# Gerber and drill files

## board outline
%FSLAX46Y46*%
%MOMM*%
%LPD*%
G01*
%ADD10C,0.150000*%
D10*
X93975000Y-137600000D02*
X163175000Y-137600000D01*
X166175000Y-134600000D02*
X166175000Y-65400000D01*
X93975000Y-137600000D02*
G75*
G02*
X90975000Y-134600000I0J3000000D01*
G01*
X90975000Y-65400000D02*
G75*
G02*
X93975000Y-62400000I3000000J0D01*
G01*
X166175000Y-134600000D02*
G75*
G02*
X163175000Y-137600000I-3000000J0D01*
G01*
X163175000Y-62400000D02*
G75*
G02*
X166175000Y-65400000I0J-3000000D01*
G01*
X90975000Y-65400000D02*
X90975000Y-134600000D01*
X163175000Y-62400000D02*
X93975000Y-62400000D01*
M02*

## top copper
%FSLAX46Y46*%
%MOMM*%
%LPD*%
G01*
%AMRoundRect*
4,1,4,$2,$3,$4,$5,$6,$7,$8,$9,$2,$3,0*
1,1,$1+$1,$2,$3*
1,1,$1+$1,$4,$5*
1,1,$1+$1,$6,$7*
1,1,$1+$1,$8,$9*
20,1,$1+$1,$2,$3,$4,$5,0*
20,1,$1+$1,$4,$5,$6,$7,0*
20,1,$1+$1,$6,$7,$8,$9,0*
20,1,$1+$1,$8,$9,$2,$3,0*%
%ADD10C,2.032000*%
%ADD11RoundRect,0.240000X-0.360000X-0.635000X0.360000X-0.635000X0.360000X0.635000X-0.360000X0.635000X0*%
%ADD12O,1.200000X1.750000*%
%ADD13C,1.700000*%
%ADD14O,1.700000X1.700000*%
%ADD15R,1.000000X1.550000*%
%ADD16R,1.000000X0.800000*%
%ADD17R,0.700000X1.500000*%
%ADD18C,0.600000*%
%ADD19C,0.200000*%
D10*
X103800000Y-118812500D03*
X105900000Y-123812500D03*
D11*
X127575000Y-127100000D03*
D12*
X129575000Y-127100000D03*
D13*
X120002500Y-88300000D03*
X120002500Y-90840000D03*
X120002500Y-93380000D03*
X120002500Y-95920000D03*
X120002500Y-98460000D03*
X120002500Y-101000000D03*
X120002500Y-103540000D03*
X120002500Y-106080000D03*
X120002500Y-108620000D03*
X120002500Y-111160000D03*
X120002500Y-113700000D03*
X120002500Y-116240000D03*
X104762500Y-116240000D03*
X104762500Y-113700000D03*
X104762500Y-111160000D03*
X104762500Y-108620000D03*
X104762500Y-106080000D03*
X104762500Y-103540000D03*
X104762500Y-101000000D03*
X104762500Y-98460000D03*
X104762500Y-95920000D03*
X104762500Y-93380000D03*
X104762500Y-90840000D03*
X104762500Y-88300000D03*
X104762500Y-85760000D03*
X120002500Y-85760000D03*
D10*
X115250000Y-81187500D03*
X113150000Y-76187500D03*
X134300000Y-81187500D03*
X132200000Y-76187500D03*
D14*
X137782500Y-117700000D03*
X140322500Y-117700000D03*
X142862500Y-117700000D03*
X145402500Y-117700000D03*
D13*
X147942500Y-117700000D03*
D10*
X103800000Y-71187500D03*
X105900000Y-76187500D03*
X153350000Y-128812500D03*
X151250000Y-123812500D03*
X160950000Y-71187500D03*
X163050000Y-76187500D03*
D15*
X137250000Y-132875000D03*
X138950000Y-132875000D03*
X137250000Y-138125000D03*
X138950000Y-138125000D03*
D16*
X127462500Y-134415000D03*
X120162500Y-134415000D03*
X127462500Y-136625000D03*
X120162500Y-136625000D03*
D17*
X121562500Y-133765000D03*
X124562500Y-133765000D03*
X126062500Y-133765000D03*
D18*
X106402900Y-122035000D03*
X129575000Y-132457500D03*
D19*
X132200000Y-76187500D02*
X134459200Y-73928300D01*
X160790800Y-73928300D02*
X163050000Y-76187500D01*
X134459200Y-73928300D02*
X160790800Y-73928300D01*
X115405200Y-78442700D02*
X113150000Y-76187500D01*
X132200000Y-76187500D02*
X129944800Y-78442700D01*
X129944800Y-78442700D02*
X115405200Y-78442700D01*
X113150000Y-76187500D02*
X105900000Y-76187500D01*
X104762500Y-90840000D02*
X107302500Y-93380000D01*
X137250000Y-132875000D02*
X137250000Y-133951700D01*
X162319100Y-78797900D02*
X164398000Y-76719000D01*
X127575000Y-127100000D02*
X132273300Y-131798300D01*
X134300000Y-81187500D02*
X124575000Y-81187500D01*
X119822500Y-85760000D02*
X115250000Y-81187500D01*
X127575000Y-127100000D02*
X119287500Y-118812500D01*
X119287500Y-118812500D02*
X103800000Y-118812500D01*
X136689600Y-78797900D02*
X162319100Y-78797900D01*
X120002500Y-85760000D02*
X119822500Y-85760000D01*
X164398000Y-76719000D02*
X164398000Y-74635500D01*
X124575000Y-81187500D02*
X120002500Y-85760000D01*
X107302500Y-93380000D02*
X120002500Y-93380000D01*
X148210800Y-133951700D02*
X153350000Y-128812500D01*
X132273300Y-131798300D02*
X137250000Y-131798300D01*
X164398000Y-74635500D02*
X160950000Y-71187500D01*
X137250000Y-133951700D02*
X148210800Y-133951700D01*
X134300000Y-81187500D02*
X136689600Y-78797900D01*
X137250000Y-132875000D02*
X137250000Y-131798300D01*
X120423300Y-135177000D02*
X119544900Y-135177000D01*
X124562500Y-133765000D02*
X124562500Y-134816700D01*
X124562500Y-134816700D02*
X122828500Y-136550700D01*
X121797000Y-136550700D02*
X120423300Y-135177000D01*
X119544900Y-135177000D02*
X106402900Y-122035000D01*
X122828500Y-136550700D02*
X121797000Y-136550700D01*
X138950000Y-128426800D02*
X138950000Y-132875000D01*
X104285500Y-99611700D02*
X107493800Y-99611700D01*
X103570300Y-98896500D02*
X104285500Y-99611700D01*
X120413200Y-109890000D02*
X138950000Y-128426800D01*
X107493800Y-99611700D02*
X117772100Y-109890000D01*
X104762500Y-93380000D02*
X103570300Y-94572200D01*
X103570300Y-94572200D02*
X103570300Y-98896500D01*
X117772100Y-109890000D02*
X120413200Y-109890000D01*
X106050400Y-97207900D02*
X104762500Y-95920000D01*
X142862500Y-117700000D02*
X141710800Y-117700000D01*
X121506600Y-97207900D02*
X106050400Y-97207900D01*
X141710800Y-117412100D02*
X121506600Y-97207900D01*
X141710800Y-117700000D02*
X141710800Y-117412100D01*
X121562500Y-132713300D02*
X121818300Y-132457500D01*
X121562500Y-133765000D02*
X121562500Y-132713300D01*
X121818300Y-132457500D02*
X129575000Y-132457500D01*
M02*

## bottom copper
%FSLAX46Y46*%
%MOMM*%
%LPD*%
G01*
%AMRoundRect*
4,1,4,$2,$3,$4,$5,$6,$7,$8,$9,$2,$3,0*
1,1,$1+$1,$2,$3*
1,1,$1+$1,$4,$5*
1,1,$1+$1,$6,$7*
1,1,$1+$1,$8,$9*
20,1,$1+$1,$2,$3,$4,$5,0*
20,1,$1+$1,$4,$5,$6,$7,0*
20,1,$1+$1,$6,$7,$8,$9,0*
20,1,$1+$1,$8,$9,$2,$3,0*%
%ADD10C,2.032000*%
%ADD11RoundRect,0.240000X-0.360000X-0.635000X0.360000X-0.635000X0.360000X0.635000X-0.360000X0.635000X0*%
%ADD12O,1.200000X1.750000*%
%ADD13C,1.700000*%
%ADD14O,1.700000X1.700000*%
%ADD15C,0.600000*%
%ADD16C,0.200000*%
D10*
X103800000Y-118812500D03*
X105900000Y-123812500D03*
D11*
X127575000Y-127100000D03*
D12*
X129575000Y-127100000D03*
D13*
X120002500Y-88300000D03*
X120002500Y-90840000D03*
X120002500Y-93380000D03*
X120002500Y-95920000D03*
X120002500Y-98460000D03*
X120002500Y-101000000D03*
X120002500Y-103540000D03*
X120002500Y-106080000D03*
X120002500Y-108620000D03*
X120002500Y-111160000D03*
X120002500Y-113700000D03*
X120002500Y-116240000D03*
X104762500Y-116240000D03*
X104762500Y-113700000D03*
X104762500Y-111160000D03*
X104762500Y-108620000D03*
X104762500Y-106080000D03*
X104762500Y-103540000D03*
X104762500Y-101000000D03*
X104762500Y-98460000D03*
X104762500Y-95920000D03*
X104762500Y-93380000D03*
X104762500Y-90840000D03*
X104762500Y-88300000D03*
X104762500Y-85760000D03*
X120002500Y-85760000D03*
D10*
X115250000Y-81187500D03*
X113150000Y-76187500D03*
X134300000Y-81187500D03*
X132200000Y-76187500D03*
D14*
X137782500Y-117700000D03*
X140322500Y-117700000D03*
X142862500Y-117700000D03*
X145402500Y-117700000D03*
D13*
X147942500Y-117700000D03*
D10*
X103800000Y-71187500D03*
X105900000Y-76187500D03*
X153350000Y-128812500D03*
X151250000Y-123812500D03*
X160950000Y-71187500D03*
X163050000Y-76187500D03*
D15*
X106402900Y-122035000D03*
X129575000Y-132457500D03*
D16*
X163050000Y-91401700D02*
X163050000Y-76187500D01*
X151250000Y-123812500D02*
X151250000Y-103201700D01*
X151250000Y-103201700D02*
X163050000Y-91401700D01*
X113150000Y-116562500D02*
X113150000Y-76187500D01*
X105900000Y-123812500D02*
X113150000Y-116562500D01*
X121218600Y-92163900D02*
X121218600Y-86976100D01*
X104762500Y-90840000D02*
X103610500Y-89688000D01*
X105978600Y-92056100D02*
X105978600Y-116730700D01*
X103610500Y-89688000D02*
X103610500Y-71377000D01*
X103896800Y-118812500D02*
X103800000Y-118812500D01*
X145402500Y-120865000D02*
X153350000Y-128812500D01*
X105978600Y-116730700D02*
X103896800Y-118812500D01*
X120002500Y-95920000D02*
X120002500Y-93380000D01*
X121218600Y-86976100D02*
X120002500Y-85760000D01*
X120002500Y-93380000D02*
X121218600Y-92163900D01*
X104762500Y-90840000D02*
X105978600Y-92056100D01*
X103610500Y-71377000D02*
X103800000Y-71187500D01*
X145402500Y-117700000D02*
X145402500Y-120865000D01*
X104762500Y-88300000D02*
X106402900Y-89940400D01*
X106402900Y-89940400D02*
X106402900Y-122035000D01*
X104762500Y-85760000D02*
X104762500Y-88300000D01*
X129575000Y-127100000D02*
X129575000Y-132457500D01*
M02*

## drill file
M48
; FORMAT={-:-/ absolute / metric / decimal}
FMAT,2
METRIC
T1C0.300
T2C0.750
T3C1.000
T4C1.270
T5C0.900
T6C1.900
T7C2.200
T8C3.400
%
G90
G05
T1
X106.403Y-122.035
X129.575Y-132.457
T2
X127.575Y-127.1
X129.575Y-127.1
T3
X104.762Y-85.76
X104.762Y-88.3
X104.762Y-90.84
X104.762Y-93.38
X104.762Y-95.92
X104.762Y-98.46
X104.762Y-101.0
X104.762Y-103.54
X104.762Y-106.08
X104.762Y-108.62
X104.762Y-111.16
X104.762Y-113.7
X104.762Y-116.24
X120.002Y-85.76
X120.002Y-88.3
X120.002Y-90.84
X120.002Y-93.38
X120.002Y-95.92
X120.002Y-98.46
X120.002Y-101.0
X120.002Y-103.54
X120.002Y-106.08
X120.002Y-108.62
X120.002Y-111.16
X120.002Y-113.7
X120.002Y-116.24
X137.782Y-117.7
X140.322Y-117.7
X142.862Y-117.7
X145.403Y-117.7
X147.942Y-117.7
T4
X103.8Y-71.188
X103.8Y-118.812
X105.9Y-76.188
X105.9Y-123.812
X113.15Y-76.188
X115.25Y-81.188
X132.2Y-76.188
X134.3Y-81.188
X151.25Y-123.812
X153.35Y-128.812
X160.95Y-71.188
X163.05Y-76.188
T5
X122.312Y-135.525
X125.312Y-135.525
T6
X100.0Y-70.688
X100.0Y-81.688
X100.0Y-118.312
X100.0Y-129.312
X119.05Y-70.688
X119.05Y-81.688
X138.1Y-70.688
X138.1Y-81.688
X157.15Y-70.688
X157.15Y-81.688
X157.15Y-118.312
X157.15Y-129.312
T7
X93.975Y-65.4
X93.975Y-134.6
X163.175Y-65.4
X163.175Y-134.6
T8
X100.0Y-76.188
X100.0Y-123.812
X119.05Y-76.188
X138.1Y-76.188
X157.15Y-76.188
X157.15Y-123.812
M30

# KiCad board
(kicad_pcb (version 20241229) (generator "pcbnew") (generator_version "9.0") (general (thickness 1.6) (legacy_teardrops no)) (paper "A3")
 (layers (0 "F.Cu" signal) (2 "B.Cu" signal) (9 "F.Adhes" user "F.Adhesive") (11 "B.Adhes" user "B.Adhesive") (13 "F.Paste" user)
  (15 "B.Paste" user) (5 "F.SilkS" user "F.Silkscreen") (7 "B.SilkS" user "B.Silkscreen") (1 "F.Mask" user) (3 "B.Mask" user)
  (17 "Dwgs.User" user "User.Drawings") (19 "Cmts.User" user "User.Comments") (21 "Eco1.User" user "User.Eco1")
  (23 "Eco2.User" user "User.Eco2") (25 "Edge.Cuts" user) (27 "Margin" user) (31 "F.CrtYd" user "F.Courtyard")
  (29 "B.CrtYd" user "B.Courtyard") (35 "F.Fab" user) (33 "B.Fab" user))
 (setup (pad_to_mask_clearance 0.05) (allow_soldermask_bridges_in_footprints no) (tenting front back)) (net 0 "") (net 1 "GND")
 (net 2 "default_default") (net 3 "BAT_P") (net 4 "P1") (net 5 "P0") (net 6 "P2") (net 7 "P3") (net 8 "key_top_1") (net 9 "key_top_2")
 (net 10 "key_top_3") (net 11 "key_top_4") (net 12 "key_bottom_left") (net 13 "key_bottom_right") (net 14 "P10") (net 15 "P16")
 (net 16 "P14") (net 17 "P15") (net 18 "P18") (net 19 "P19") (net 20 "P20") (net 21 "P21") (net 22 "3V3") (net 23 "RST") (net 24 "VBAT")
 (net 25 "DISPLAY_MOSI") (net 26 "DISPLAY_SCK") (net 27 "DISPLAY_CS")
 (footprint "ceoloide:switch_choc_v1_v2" (layer "F.Cu") (at 100 123.8125 -90)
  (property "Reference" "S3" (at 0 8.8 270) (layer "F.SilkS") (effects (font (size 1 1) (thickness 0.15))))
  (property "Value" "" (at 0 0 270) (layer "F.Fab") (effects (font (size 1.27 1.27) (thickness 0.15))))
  (pad "" np_thru_hole circle (at -5.5 0 270) (size 1.9 1.9) (drill 1.9) (layers "*.Cu" "*.Mask"))
  (pad "" np_thru_hole circle (at 0 0 270) (size 3.4 3.4) (drill 3.4) (layers "*.Cu" "*.Mask"))
  (pad "" np_thru_hole circle (at 5.5 0 270) (size 1.9 1.9) (drill 1.9) (layers "*.Cu" "*.Mask"))
  (pad "1" thru_hole circle (at -5 -3.8 105) (size 2.032 2.032) (drill 1.27) (layers "*.Cu" "*.Mask") (remove_unused_layers no)
   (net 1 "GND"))
  (pad "2" thru_hole circle (at 0 -5.9 105) (size 2.032 2.032) (drill 1.27) (layers "*.Cu" "*.Mask") (remove_unused_layers no)
   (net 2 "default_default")))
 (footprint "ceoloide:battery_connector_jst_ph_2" (layer "F.Cu") (at 128.575 127.1)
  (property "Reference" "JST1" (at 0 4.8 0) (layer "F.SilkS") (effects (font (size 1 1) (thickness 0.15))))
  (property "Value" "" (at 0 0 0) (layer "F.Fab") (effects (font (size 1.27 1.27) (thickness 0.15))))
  (pad "1" thru_hole roundrect (at -1 0) (size 1.2 1.75) (drill 0.75) (layers "*.Cu" "*.Mask") (remove_unused_layers no)
   (roundrect_rratio 0.2) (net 1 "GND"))
  (pad "2" thru_hole oval (at 1 0) (size 1.2 1.75) (drill 0.75) (layers "*.Cu" "*.Mask") (remove_unused_layers no) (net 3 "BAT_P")))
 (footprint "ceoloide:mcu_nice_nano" (layer "F.Cu") (at 112.3825 101)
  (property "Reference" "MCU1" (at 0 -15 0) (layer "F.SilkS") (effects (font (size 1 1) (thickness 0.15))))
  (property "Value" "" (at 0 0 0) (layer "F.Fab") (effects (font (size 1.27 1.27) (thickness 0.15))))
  (pad "1" thru_hole circle (at 7.62 -12.7) (size 1.7 1.7) (drill 1) (layers "*.Cu" "*.Mask") (remove_unused_layers no) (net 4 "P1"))
  (pad "2" thru_hole circle (at 7.62 -10.16) (size 1.7 1.7) (drill 1) (layers "*.Cu" "*.Mask") (remove_unused_layers no) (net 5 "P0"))
  (pad "3" thru_hole circle (at 7.62 -7.62) (size 1.7 1.7) (drill 1) (layers "*.Cu" "*.Mask") (remove_unused_layers no) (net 1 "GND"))
  (pad "4" thru_hole circle (at 7.62 -5.08) (size 1.7 1.7) (drill 1) (layers "*.Cu" "*.Mask") (remove_unused_layers no) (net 1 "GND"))
  (pad "5" thru_hole circle (at 7.62 -2.54) (size 1.7 1.7) (drill 1) (layers "*.Cu" "*.Mask") (remove_unused_layers no) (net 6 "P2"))
  (pad "6" thru_hole circle (at 7.62 0) (size 1.7 1.7) (drill 1) (layers "*.Cu" "*.Mask") (remove_unused_layers no) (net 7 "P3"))
  (pad "7" thru_hole circle (at 7.62 2.54) (size 1.7 1.7) (drill 1) (layers "*.Cu" "*.Mask") (remove_unused_layers no) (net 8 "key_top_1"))
  (pad "8" thru_hole circle (at 7.62 5.08) (size 1.7 1.7) (drill 1) (layers "*.Cu" "*.Mask") (remove_unused_layers no) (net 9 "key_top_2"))
  (pad "9" thru_hole circle (at 7.62 7.62) (size 1.7 1.7) (drill 1) (layers "*.Cu" "*.Mask") (remove_unused_layers no) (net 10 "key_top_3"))
  (pad "10" thru_hole circle (at 7.62 10.16) (size 1.7 1.7) (drill 1) (layers "*.Cu" "*.Mask") (remove_unused_layers no)
   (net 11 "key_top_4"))
  (pad "11" thru_hole circle (at 7.62 12.7) (size 1.7 1.7) (drill 1) (layers "*.Cu" "*.Mask") (remove_unused_layers no)
   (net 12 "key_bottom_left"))
  (pad "12" thru_hole circle (at 7.62 15.24) (size 1.7 1.7) (drill 1) (layers "*.Cu" "*.Mask") (remove_unused_layers no)
   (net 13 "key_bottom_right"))
  (pad "13" thru_hole circle (at -7.62 15.24) (size 1.7 1.7) (drill 1) (layers "*.Cu" "*.Mask") (remove_unused_layers no) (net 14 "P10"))
  (pad "14" thru_hole circle (at -7.62 12.7) (size 1.7 1.7) (drill 1) (layers "*.Cu" "*.Mask") (remove_unused_layers no) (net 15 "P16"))
  (pad "15" thru_hole circle (at -7.62 10.16) (size 1.7 1.7) (drill 1) (layers "*.Cu" "*.Mask") (remove_unused_layers no) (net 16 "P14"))
  (pad "16" thru_hole circle (at -7.62 7.62) (size 1.7 1.7) (drill 1) (layers "*.Cu" "*.Mask") (remove_unused_layers no) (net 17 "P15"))
  (pad "17" thru_hole circle (at -7.62 5.08) (size 1.7 1.7) (drill 1) (layers "*.Cu" "*.Mask") (remove_unused_layers no) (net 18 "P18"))
  (pad "18" thru_hole circle (at -7.62 2.54) (size 1.7 1.7) (drill 1) (layers "*.Cu" "*.Mask") (remove_unused_layers no) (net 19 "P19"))
  (pad "19" thru_hole circle (at -7.62 0) (size 1.7 1.7) (drill 1) (layers "*.Cu" "*.Mask") (remove_unused_layers no) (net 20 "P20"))
  (pad "20" thru_hole circle (at -7.62 -2.54) (size 1.7 1.7) (drill 1) (layers "*.Cu" "*.Mask") (remove_unused_layers no) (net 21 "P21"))
  (pad "21" thru_hole circle (at -7.62 -5.08) (size 1.7 1.7) (drill 1) (layers "*.Cu" "*.Mask") (remove_unused_layers no) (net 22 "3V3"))
  (pad "22" thru_hole circle (at -7.62 -7.62) (size 1.7 1.7) (drill 1) (layers "*.Cu" "*.Mask") (remove_unused_layers no) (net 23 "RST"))
  (pad "23" thru_hole circle (at -7.62 -10.16) (size 1.7 1.7) (drill 1) (layers "*.Cu" "*.Mask") (remove_unused_layers no) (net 1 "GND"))
  (pad "24" thru_hole circle (at -7.62 -12.7) (size 1.7 1.7) (drill 1) (layers "*.Cu" "*.Mask") (remove_unused_layers no) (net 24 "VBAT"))
  (pad "25" thru_hole circle (at -7.62 -15.24) (size 1.7 1.7) (drill 1) (layers "*.Cu" "*.Mask") (remove_unused_layers no) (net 24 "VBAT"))
  (pad "26" thru_hole circle (at 7.62 -15.24) (size 1.7 1.7) (drill 1) (layers "*.Cu" "*.Mask") (remove_unused_layers no) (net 1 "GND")))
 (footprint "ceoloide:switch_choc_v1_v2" (layer "F.Cu") (at 119.05 76.1875 90)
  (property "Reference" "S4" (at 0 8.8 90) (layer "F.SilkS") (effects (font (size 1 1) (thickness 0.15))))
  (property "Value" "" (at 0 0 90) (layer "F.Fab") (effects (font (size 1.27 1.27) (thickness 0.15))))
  (pad "" np_thru_hole circle (at -5.5 0 90) (size 1.9 1.9) (drill 1.9) (layers "*.Cu" "*.Mask"))
  (pad "" np_thru_hole circle (at 0 0 90) (size 3.4 3.4) (drill 3.4) (layers "*.Cu" "*.Mask"))
  (pad "" np_thru_hole circle (at 5.5 0 90) (size 1.9 1.9) (drill 1.9) (layers "*.Cu" "*.Mask"))
  (pad "1" thru_hole circle (at -5 -3.8 285) (size 2.032 2.032) (drill 1.27) (layers "*.Cu" "*.Mask") (remove_unused_layers no)
   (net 1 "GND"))
  (pad "2" thru_hole circle (at 0 -5.9 285) (size 2.032 2.032) (drill 1.27) (layers "*.Cu" "*.Mask") (remove_unused_layers no)
   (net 2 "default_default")))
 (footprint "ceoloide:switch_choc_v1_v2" (layer "F.Cu") (at 138.1 76.1875 90)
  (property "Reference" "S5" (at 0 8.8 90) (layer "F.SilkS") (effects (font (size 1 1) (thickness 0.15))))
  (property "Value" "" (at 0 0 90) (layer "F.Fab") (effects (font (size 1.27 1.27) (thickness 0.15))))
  (pad "" np_thru_hole circle (at -5.5 0 90) (size 1.9 1.9) (drill 1.9) (layers "*.Cu" "*.Mask"))
  (pad "" np_thru_hole circle (at 0 0 90) (size 3.4 3.4) (drill 3.4) (layers "*.Cu" "*.Mask"))
  (pad "" np_thru_hole circle (at 5.5 0 90) (size 1.9 1.9) (drill 1.9) (layers "*.Cu" "*.Mask"))
  (pad "1" thru_hole circle (at -5 -3.8 285) (size 2.032 2.032) (drill 1.27) (layers "*.Cu" "*.Mask") (remove_unused_layers no)
   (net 1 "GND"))
  (pad "2" thru_hole circle (at 0 -5.9 285) (size 2.032 2.032) (drill 1.27) (layers "*.Cu" "*.Mask") (remove_unused_layers no)
   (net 2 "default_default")))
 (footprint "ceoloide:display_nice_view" (layer "F.Cu") (at 142.8625 101)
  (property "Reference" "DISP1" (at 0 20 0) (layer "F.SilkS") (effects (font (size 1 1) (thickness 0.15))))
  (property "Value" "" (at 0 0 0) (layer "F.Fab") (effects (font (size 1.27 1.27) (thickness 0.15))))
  (pad "1" thru_hole oval (at -5.08 16.7 270) (size 1.7 1.7) (drill 1) (layers "*.Cu" "*.Mask") (remove_unused_layers no)
   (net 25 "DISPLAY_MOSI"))
  (pad "2" thru_hole oval (at -2.54 16.7 270) (size 1.7 1.7) (drill 1) (layers "*.Cu" "*.Mask") (remove_unused_layers no)
   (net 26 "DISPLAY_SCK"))
  (pad "3" thru_hole oval (at 0 16.7 270) (size 1.7 1.7) (drill 1) (layers "*.Cu" "*.Mask") (remove_unused_layers no) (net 22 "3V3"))
  (pad "4" thru_hole oval (at 2.54 16.7 270) (size 1.7 1.7) (drill 1) (layers "*.Cu" "*.Mask") (remove_unused_layers no) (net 1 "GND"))
  (pad "5" thru_hole circle (at 5.08 16.7 270) (size 1.7 1.7) (drill 1) (layers "*.Cu" "*.Mask") (remove_unused_layers no)
   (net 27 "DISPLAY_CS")))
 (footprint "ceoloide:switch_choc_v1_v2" (layer "F.Cu") (at 100 76.1875 -90)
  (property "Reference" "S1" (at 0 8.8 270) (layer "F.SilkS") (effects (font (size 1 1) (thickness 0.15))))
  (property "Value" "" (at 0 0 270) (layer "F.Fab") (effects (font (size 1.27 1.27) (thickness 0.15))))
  (pad "" np_thru_hole circle (at -5.5 0 270) (size 1.9 1.9) (drill 1.9) (layers "*.Cu" "*.Mask"))
  (pad "" np_thru_hole circle (at 0 0 270) (size 3.4 3.4) (drill 3.4) (layers "*.Cu" "*.Mask"))
  (pad "" np_thru_hole circle (at 5.5 0 270) (size 1.9 1.9) (drill 1.9) (layers "*.Cu" "*.Mask"))
  (pad "1" thru_hole circle (at -5 -3.8 105) (size 2.032 2.032) (drill 1.27) (layers "*.Cu" "*.Mask") (remove_unused_layers no)
   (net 1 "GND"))
  (pad "2" thru_hole circle (at 0 -5.9 105) (size 2.032 2.032) (drill 1.27) (layers "*.Cu" "*.Mask") (remove_unused_layers no)
   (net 2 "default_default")))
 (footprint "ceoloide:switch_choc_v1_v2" (layer "F.Cu") (at 157.15 123.8125 90)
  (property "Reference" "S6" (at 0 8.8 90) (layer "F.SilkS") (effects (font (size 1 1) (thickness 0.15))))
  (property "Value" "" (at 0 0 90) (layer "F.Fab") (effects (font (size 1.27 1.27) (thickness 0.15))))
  (pad "" np_thru_hole circle (at -5.5 0 90) (size 1.9 1.9) (drill 1.9) (layers "*.Cu" "*.Mask"))
  (pad "" np_thru_hole circle (at 0 0 90) (size 3.4 3.4) (drill 3.4) (layers "*.Cu" "*.Mask"))
  (pad "" np_thru_hole circle (at 5.5 0 90) (size 1.9 1.9) (drill 1.9) (layers "*.Cu" "*.Mask"))
  (pad "1" thru_hole circle (at -5 -3.8 285) (size 2.032 2.032) (drill 1.27) (layers "*.Cu" "*.Mask") (remove_unused_layers no)
   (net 1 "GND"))
  (pad "2" thru_hole circle (at 0 -5.9 285) (size 2.032 2.032) (drill 1.27) (layers "*.Cu" "*.Mask") (remove_unused_layers no)
   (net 2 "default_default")))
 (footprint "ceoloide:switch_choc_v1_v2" (layer "F.Cu") (at 157.15 76.1875 -90)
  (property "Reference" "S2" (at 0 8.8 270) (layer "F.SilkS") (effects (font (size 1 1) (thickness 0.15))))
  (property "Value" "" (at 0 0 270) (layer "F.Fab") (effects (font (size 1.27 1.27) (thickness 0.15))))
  (pad "" np_thru_hole circle (at -5.5 0 270) (size 1.9 1.9) (drill 1.9) (layers "*.Cu" "*.Mask"))
  (pad "" np_thru_hole circle (at 0 0 270) (size 3.4 3.4) (drill 3.4) (layers "*.Cu" "*.Mask"))
  (pad "" np_thru_hole circle (at 5.5 0 270) (size 1.9 1.9) (drill 1.9) (layers "*.Cu" "*.Mask"))
  (pad "1" thru_hole circle (at -5 -3.8 105) (size 2.032 2.032) (drill 1.27) (layers "*.Cu" "*.Mask") (remove_unused_layers no)
   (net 1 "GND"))
  (pad "2" thru_hole circle (at 0 -5.9 105) (size 2.032 2.032) (drill 1.27) (layers "*.Cu" "*.Mask") (remove_unused_layers no)
   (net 2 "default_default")))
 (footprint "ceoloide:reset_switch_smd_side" (layer "F.Cu") (at 138.1 135.5 90)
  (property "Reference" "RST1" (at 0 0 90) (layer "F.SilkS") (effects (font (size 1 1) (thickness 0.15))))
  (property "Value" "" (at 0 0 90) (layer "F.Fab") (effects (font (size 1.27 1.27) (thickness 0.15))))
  (pad "1" smd rect (at 2.625 -0.85 270) (size 1.55 1) (layers "F.Cu" "F.Mask" "F.Paste") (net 1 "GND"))
  (pad "2" smd rect (at 2.625 0.85 270) (size 1.55 1) (layers "F.Cu" "F.Mask" "F.Paste") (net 23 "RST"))
  (pad "3" smd rect (at -2.625 -0.85 270) (size 1.55 1) (layers "F.Cu" "F.Mask" "F.Paste") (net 1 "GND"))
  (pad "4" smd rect (at -2.625 0.85 270) (size 1.55 1) (layers "F.Cu" "F.Mask" "F.Paste") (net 23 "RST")))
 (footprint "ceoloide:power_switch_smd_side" (layer "F.Cu") (at 123.8125 135.5 -90)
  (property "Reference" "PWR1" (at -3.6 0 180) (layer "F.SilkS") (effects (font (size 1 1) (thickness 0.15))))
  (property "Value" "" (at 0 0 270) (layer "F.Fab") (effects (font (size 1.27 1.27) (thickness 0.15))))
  (pad "" smd rect (at -1.085 -3.65) (size 1 0.8) (layers "F.Cu" "F.Mask" "F.Paste"))
  (pad "" smd rect (at -1.085 3.65) (size 1 0.8) (layers "F.Cu" "F.Mask" "F.Paste"))
  (pad "" np_thru_hole circle (at 0.025 -1.5) (size 0.9 0.9) (drill 0.9) (layers "*.Cu" "*.Mask"))
  (pad "" np_thru_hole circle (at 0.025 1.5) (size 0.9 0.9) (drill 0.9) (layers "*.Cu" "*.Mask"))
  (pad "" smd rect (at 1.125 -3.65) (size 1 0.8) (layers "F.Cu" "F.Mask" "F.Paste"))
  (pad "" smd rect (at 1.125 3.65) (size 1 0.8) (layers "F.Cu" "F.Mask" "F.Paste"))
  (pad "1" smd rect (at -1.735 2.25) (size 0.7 1.5) (layers "F.Cu" "F.Mask" "F.Paste") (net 3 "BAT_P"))
  (pad "2" smd rect (at -1.735 -0.75) (size 0.7 1.5) (layers "F.Cu" "F.Mask" "F.Paste") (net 24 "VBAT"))
  (pad "3" smd rect (at -1.735 -2.25) (size 0.7 1.5) (layers "F.Cu" "F.Mask" "F.Paste")))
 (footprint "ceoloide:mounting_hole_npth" (layer "B.Cu") (at 93.975 134.6)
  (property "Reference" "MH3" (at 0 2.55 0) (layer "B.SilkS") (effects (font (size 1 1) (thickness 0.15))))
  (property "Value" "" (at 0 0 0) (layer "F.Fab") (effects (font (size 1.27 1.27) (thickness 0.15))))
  (pad "" np_thru_hole circle (at 0 0) (size 2.2 2.2) (drill 2.2) (layers "*.Cu" "*.Mask")))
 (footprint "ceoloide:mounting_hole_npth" (layer "B.Cu") (at 93.975 65.4)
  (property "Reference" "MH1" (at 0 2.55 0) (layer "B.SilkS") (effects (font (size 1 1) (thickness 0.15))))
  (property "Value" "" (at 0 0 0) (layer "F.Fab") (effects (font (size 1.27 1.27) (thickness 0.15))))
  (pad "" np_thru_hole circle (at 0 0) (size 2.2 2.2) (drill 2.2) (layers "*.Cu" "*.Mask")))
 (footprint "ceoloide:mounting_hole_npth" (layer "B.Cu") (at 163.175 134.6)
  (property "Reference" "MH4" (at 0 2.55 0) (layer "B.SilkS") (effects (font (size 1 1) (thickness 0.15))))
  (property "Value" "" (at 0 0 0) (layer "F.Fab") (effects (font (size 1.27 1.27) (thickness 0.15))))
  (pad "" np_thru_hole circle (at 0 0) (size 2.2 2.2) (drill 2.2) (layers "*.Cu" "*.Mask")))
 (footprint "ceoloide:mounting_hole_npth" (layer "B.Cu") (at 163.175 65.4)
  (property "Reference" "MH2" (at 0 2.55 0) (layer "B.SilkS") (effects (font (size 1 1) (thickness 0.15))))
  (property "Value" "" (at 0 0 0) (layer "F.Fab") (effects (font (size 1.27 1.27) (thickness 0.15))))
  (pad "" np_thru_hole circle (at 0 0) (size 2.2 2.2) (drill 2.2) (layers "*.Cu" "*.Mask")))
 (gr_line (start 93.975 137.6) (end 163.175 137.6) (stroke (width 0.15) (type default)) (layer "Edge.Cuts"))
 (gr_line (start 166.175 134.6) (end 166.175 65.4) (stroke (width 0.15) (type default)) (layer "Edge.Cuts"))
 (gr_arc (start 93.975 137.6) (mid 91.85368 136.72132) (end 90.975 134.6) (stroke (width 0.15) (type default)) (layer "Edge.Cuts"))
 (gr_arc (start 90.975 65.4) (mid 91.85368 63.27868) (end 93.975 62.4) (stroke (width 0.15) (type default)) (layer "Edge.Cuts"))
 (gr_arc (start 166.175 134.6) (mid 165.29632 136.72132) (end 163.175 137.6) (stroke (width 0.15) (type default)) (layer "Edge.Cuts"))
 (gr_arc (start 163.175 62.4) (mid 165.29632 63.27868) (end 166.175 65.4) (stroke (width 0.15) (type default)) (layer "Edge.Cuts"))
 (gr_line (start 90.975 65.4) (end 90.975 134.6) (stroke (width 0.15) (type default)) (layer "Edge.Cuts"))
 (gr_line (start 163.175 62.4) (end 93.975 62.4) (stroke (width 0.15) (type default)) (layer "Edge.Cuts"))
 (segment (start 132.2 76.1875) (end 134.4592 73.9283) (width 0.2) (layer "F.Cu") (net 2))
 (segment (start 160.7908 73.9283) (end 163.05 76.1875) (width 0.2) (layer "F.Cu") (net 2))
 (segment (start 134.4592 73.9283) (end 160.7908 73.9283) (width 0.2) (layer "F.Cu") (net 2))
 (segment (start 115.4052 78.4427) (end 113.15 76.1875) (width 0.2) (layer "F.Cu") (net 2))
 (segment (start 132.2 76.1875) (end 129.9448 78.4427) (width 0.2) (layer "F.Cu") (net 2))
 (segment (start 129.9448 78.4427) (end 115.4052 78.4427) (width 0.2) (layer "F.Cu") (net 2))
 (segment (start 113.15 76.1875) (end 105.9 76.1875) (width 0.2) (layer "F.Cu") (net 2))
 (segment (start 163.05 91.4017) (end 163.05 76.1875) (width 0.2) (layer "B.Cu") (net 2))
 (segment (start 151.25 123.8125) (end 151.25 103.2017) (width 0.2) (layer "B.Cu") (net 2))
 (segment (start 151.25 103.2017) (end 163.05 91.4017) (width 0.2) (layer "B.Cu") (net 2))
 (segment (start 113.15 116.5625) (end 113.15 76.1875) (width 0.2) (layer "B.Cu") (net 2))
 (segment (start 105.9 123.8125) (end 113.15 116.5625) (width 0.2) (layer "B.Cu") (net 2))
 (segment (start 104.7625 90.84) (end 107.3025 93.38) (width 0.2) (layer "F.Cu") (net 1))
 (segment (start 137.25 132.875) (end 137.25 133.9517) (width 0.2) (layer "F.Cu") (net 1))
 (segment (start 162.3191 78.7979) (end 164.398 76.719) (width 0.2) (layer "F.Cu") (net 1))
 (segment (start 127.575 127.1) (end 132.2733 131.7983) (width 0.2) (layer "F.Cu") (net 1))
 (segment (start 134.3 81.1875) (end 124.575 81.1875) (width 0.2) (layer "F.Cu") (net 1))
 (segment (start 119.8225 85.76) (end 115.25 81.1875) (width 0.2) (layer "F.Cu") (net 1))
 (segment (start 127.575 127.1) (end 119.2875 118.8125) (width 0.2) (layer "F.Cu") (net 1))
 (segment (start 119.2875 118.8125) (end 103.8 118.8125) (width 0.2) (layer "F.Cu") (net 1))
 (segment (start 136.6896 78.7979) (end 162.3191 78.7979) (width 0.2) (layer "F.Cu") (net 1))
 (segment (start 120.0025 85.76) (end 119.8225 85.76) (width 0.2) (layer "F.Cu") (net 1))
 (segment (start 164.398 76.719) (end 164.398 74.6355) (width 0.2) (layer "F.Cu") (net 1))
 (segment (start 124.575 81.1875) (end 120.0025 85.76) (width 0.2) (layer "F.Cu") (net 1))
 (segment (start 107.3025 93.38) (end 120.0025 93.38) (width 0.2) (layer "F.Cu") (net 1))
 (segment (start 148.2108 133.9517) (end 153.35 128.8125) (width 0.2) (layer "F.Cu") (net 1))
 (segment (start 132.2733 131.7983) (end 137.25 131.7983) (width 0.2) (layer "F.Cu") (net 1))
 (segment (start 164.398 74.6355) (end 160.95 71.1875) (width 0.2) (layer "F.Cu") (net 1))
 (segment (start 137.25 133.9517) (end 148.2108 133.9517) (width 0.2) (layer "F.Cu") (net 1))
 (segment (start 134.3 81.1875) (end 136.6896 78.7979) (width 0.2) (layer "F.Cu") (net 1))
 (segment (start 137.25 132.875) (end 137.25 131.7983) (width 0.2) (layer "F.Cu") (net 1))
 (segment (start 121.2186 92.1639) (end 121.2186 86.9761) (width 0.2) (layer "B.Cu") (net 1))
 (segment (start 104.7625 90.84) (end 103.6105 89.688) (width 0.2) (layer "B.Cu") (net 1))
 (segment (start 105.9786 92.0561) (end 105.9786 116.7307) (width 0.2) (layer "B.Cu") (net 1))
 (segment (start 103.6105 89.688) (end 103.6105 71.377) (width 0.2) (layer "B.Cu") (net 1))
 (segment (start 103.8968 118.8125) (end 103.8 118.8125) (width 0.2) (layer "B.Cu") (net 1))
 (segment (start 145.4025 120.865) (end 153.35 128.8125) (width 0.2) (layer "B.Cu") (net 1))
 (segment (start 105.9786 116.7307) (end 103.8968 118.8125) (width 0.2) (layer "B.Cu") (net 1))
 (segment (start 120.0025 95.92) (end 120.0025 93.38) (width 0.2) (layer "B.Cu") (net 1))
 (segment (start 121.2186 86.9761) (end 120.0025 85.76) (width 0.2) (layer "B.Cu") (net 1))
 (segment (start 120.0025 93.38) (end 121.2186 92.1639) (width 0.2) (layer "B.Cu") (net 1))
 (segment (start 104.7625 90.84) (end 105.9786 92.0561) (width 0.2) (layer "B.Cu") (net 1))
 (segment (start 103.6105 71.377) (end 103.8 71.1875) (width 0.2) (layer "B.Cu") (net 1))
 (segment (start 145.4025 117.7) (end 145.4025 120.865) (width 0.2) (layer "B.Cu") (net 1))
 (segment (start 120.4233 135.177) (end 119.5449 135.177) (width 0.2) (layer "F.Cu") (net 24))
 (segment (start 124.5625 133.765) (end 124.5625 134.8167) (width 0.2) (layer "F.Cu") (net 24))
 (segment (start 124.5625 134.8167) (end 122.8285 136.5507) (width 0.2) (layer "F.Cu") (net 24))
 (segment (start 121.797 136.5507) (end 120.4233 135.177) (width 0.2) (layer "F.Cu") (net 24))
 (segment (start 119.5449 135.177) (end 106.4029 122.035) (width 0.2) (layer "F.Cu") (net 24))
 (segment (start 122.8285 136.5507) (end 121.797 136.5507) (width 0.2) (layer "F.Cu") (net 24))
 (via (at 106.4029 122.035) (size 0.6) (drill 0.3) (layers "F.Cu" "B.Cu") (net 24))
 (segment (start 104.7625 88.3) (end 106.4029 89.9404) (width 0.2) (layer "B.Cu") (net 24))
 (segment (start 106.4029 89.9404) (end 106.4029 122.035) (width 0.2) (layer "B.Cu") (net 24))
 (segment (start 104.7625 85.76) (end 104.7625 88.3) (width 0.2) (layer "B.Cu") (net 24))
 (segment (start 138.95 128.4268) (end 138.95 132.875) (width 0.2) (layer "F.Cu") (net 23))
 (segment (start 104.2855 99.6117) (end 107.4938 99.6117) (width 0.2) (layer "F.Cu") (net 23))
 (segment (start 103.5703 98.8965) (end 104.2855 99.6117) (width 0.2) (layer "F.Cu") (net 23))
 (segment (start 120.4132 109.89) (end 138.95 128.4268) (width 0.2) (layer "F.Cu") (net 23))
 (segment (start 107.4938 99.6117) (end 117.7721 109.89) (width 0.2) (layer "F.Cu") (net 23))
 (segment (start 104.7625 93.38) (end 103.5703 94.5722) (width 0.2) (layer "F.Cu") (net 23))
 (segment (start 103.5703 94.5722) (end 103.5703 98.8965) (width 0.2) (layer "F.Cu") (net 23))
 (segment (start 117.7721 109.89) (end 120.4132 109.89) (width 0.2) (layer "F.Cu") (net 23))
 (segment (start 106.0504 97.2079) (end 104.7625 95.92) (width 0.2) (layer "F.Cu") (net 22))
 (segment (start 142.8625 117.7) (end 141.7108 117.7) (width 0.2) (layer "F.Cu") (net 22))
 (segment (start 121.5066 97.2079) (end 106.0504 97.2079) (width 0.2) (layer "F.Cu") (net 22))
 (segment (start 141.7108 117.4121) (end 121.5066 97.2079) (width 0.2) (layer "F.Cu") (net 22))
 (segment (start 141.7108 117.7) (end 141.7108 117.4121) (width 0.2) (layer "F.Cu") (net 22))
 (segment (start 121.5625 132.7133) (end 121.8183 132.4575) (width 0.2) (layer "F.Cu") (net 3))
 (segment (start 121.5625 133.765) (end 121.5625 132.7133) (width 0.2) (layer "F.Cu") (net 3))
 (segment (start 121.8183 132.4575) (end 129.575 132.4575) (width 0.2) (layer "F.Cu") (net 3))
 (via (at 129.575 132.4575) (size 0.6) (drill 0.3) (layers "F.Cu" "B.Cu") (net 3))
 (segment (start 129.575 127.1) (end 129.575 132.4575) (width 0.2) (layer "B.Cu") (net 3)))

